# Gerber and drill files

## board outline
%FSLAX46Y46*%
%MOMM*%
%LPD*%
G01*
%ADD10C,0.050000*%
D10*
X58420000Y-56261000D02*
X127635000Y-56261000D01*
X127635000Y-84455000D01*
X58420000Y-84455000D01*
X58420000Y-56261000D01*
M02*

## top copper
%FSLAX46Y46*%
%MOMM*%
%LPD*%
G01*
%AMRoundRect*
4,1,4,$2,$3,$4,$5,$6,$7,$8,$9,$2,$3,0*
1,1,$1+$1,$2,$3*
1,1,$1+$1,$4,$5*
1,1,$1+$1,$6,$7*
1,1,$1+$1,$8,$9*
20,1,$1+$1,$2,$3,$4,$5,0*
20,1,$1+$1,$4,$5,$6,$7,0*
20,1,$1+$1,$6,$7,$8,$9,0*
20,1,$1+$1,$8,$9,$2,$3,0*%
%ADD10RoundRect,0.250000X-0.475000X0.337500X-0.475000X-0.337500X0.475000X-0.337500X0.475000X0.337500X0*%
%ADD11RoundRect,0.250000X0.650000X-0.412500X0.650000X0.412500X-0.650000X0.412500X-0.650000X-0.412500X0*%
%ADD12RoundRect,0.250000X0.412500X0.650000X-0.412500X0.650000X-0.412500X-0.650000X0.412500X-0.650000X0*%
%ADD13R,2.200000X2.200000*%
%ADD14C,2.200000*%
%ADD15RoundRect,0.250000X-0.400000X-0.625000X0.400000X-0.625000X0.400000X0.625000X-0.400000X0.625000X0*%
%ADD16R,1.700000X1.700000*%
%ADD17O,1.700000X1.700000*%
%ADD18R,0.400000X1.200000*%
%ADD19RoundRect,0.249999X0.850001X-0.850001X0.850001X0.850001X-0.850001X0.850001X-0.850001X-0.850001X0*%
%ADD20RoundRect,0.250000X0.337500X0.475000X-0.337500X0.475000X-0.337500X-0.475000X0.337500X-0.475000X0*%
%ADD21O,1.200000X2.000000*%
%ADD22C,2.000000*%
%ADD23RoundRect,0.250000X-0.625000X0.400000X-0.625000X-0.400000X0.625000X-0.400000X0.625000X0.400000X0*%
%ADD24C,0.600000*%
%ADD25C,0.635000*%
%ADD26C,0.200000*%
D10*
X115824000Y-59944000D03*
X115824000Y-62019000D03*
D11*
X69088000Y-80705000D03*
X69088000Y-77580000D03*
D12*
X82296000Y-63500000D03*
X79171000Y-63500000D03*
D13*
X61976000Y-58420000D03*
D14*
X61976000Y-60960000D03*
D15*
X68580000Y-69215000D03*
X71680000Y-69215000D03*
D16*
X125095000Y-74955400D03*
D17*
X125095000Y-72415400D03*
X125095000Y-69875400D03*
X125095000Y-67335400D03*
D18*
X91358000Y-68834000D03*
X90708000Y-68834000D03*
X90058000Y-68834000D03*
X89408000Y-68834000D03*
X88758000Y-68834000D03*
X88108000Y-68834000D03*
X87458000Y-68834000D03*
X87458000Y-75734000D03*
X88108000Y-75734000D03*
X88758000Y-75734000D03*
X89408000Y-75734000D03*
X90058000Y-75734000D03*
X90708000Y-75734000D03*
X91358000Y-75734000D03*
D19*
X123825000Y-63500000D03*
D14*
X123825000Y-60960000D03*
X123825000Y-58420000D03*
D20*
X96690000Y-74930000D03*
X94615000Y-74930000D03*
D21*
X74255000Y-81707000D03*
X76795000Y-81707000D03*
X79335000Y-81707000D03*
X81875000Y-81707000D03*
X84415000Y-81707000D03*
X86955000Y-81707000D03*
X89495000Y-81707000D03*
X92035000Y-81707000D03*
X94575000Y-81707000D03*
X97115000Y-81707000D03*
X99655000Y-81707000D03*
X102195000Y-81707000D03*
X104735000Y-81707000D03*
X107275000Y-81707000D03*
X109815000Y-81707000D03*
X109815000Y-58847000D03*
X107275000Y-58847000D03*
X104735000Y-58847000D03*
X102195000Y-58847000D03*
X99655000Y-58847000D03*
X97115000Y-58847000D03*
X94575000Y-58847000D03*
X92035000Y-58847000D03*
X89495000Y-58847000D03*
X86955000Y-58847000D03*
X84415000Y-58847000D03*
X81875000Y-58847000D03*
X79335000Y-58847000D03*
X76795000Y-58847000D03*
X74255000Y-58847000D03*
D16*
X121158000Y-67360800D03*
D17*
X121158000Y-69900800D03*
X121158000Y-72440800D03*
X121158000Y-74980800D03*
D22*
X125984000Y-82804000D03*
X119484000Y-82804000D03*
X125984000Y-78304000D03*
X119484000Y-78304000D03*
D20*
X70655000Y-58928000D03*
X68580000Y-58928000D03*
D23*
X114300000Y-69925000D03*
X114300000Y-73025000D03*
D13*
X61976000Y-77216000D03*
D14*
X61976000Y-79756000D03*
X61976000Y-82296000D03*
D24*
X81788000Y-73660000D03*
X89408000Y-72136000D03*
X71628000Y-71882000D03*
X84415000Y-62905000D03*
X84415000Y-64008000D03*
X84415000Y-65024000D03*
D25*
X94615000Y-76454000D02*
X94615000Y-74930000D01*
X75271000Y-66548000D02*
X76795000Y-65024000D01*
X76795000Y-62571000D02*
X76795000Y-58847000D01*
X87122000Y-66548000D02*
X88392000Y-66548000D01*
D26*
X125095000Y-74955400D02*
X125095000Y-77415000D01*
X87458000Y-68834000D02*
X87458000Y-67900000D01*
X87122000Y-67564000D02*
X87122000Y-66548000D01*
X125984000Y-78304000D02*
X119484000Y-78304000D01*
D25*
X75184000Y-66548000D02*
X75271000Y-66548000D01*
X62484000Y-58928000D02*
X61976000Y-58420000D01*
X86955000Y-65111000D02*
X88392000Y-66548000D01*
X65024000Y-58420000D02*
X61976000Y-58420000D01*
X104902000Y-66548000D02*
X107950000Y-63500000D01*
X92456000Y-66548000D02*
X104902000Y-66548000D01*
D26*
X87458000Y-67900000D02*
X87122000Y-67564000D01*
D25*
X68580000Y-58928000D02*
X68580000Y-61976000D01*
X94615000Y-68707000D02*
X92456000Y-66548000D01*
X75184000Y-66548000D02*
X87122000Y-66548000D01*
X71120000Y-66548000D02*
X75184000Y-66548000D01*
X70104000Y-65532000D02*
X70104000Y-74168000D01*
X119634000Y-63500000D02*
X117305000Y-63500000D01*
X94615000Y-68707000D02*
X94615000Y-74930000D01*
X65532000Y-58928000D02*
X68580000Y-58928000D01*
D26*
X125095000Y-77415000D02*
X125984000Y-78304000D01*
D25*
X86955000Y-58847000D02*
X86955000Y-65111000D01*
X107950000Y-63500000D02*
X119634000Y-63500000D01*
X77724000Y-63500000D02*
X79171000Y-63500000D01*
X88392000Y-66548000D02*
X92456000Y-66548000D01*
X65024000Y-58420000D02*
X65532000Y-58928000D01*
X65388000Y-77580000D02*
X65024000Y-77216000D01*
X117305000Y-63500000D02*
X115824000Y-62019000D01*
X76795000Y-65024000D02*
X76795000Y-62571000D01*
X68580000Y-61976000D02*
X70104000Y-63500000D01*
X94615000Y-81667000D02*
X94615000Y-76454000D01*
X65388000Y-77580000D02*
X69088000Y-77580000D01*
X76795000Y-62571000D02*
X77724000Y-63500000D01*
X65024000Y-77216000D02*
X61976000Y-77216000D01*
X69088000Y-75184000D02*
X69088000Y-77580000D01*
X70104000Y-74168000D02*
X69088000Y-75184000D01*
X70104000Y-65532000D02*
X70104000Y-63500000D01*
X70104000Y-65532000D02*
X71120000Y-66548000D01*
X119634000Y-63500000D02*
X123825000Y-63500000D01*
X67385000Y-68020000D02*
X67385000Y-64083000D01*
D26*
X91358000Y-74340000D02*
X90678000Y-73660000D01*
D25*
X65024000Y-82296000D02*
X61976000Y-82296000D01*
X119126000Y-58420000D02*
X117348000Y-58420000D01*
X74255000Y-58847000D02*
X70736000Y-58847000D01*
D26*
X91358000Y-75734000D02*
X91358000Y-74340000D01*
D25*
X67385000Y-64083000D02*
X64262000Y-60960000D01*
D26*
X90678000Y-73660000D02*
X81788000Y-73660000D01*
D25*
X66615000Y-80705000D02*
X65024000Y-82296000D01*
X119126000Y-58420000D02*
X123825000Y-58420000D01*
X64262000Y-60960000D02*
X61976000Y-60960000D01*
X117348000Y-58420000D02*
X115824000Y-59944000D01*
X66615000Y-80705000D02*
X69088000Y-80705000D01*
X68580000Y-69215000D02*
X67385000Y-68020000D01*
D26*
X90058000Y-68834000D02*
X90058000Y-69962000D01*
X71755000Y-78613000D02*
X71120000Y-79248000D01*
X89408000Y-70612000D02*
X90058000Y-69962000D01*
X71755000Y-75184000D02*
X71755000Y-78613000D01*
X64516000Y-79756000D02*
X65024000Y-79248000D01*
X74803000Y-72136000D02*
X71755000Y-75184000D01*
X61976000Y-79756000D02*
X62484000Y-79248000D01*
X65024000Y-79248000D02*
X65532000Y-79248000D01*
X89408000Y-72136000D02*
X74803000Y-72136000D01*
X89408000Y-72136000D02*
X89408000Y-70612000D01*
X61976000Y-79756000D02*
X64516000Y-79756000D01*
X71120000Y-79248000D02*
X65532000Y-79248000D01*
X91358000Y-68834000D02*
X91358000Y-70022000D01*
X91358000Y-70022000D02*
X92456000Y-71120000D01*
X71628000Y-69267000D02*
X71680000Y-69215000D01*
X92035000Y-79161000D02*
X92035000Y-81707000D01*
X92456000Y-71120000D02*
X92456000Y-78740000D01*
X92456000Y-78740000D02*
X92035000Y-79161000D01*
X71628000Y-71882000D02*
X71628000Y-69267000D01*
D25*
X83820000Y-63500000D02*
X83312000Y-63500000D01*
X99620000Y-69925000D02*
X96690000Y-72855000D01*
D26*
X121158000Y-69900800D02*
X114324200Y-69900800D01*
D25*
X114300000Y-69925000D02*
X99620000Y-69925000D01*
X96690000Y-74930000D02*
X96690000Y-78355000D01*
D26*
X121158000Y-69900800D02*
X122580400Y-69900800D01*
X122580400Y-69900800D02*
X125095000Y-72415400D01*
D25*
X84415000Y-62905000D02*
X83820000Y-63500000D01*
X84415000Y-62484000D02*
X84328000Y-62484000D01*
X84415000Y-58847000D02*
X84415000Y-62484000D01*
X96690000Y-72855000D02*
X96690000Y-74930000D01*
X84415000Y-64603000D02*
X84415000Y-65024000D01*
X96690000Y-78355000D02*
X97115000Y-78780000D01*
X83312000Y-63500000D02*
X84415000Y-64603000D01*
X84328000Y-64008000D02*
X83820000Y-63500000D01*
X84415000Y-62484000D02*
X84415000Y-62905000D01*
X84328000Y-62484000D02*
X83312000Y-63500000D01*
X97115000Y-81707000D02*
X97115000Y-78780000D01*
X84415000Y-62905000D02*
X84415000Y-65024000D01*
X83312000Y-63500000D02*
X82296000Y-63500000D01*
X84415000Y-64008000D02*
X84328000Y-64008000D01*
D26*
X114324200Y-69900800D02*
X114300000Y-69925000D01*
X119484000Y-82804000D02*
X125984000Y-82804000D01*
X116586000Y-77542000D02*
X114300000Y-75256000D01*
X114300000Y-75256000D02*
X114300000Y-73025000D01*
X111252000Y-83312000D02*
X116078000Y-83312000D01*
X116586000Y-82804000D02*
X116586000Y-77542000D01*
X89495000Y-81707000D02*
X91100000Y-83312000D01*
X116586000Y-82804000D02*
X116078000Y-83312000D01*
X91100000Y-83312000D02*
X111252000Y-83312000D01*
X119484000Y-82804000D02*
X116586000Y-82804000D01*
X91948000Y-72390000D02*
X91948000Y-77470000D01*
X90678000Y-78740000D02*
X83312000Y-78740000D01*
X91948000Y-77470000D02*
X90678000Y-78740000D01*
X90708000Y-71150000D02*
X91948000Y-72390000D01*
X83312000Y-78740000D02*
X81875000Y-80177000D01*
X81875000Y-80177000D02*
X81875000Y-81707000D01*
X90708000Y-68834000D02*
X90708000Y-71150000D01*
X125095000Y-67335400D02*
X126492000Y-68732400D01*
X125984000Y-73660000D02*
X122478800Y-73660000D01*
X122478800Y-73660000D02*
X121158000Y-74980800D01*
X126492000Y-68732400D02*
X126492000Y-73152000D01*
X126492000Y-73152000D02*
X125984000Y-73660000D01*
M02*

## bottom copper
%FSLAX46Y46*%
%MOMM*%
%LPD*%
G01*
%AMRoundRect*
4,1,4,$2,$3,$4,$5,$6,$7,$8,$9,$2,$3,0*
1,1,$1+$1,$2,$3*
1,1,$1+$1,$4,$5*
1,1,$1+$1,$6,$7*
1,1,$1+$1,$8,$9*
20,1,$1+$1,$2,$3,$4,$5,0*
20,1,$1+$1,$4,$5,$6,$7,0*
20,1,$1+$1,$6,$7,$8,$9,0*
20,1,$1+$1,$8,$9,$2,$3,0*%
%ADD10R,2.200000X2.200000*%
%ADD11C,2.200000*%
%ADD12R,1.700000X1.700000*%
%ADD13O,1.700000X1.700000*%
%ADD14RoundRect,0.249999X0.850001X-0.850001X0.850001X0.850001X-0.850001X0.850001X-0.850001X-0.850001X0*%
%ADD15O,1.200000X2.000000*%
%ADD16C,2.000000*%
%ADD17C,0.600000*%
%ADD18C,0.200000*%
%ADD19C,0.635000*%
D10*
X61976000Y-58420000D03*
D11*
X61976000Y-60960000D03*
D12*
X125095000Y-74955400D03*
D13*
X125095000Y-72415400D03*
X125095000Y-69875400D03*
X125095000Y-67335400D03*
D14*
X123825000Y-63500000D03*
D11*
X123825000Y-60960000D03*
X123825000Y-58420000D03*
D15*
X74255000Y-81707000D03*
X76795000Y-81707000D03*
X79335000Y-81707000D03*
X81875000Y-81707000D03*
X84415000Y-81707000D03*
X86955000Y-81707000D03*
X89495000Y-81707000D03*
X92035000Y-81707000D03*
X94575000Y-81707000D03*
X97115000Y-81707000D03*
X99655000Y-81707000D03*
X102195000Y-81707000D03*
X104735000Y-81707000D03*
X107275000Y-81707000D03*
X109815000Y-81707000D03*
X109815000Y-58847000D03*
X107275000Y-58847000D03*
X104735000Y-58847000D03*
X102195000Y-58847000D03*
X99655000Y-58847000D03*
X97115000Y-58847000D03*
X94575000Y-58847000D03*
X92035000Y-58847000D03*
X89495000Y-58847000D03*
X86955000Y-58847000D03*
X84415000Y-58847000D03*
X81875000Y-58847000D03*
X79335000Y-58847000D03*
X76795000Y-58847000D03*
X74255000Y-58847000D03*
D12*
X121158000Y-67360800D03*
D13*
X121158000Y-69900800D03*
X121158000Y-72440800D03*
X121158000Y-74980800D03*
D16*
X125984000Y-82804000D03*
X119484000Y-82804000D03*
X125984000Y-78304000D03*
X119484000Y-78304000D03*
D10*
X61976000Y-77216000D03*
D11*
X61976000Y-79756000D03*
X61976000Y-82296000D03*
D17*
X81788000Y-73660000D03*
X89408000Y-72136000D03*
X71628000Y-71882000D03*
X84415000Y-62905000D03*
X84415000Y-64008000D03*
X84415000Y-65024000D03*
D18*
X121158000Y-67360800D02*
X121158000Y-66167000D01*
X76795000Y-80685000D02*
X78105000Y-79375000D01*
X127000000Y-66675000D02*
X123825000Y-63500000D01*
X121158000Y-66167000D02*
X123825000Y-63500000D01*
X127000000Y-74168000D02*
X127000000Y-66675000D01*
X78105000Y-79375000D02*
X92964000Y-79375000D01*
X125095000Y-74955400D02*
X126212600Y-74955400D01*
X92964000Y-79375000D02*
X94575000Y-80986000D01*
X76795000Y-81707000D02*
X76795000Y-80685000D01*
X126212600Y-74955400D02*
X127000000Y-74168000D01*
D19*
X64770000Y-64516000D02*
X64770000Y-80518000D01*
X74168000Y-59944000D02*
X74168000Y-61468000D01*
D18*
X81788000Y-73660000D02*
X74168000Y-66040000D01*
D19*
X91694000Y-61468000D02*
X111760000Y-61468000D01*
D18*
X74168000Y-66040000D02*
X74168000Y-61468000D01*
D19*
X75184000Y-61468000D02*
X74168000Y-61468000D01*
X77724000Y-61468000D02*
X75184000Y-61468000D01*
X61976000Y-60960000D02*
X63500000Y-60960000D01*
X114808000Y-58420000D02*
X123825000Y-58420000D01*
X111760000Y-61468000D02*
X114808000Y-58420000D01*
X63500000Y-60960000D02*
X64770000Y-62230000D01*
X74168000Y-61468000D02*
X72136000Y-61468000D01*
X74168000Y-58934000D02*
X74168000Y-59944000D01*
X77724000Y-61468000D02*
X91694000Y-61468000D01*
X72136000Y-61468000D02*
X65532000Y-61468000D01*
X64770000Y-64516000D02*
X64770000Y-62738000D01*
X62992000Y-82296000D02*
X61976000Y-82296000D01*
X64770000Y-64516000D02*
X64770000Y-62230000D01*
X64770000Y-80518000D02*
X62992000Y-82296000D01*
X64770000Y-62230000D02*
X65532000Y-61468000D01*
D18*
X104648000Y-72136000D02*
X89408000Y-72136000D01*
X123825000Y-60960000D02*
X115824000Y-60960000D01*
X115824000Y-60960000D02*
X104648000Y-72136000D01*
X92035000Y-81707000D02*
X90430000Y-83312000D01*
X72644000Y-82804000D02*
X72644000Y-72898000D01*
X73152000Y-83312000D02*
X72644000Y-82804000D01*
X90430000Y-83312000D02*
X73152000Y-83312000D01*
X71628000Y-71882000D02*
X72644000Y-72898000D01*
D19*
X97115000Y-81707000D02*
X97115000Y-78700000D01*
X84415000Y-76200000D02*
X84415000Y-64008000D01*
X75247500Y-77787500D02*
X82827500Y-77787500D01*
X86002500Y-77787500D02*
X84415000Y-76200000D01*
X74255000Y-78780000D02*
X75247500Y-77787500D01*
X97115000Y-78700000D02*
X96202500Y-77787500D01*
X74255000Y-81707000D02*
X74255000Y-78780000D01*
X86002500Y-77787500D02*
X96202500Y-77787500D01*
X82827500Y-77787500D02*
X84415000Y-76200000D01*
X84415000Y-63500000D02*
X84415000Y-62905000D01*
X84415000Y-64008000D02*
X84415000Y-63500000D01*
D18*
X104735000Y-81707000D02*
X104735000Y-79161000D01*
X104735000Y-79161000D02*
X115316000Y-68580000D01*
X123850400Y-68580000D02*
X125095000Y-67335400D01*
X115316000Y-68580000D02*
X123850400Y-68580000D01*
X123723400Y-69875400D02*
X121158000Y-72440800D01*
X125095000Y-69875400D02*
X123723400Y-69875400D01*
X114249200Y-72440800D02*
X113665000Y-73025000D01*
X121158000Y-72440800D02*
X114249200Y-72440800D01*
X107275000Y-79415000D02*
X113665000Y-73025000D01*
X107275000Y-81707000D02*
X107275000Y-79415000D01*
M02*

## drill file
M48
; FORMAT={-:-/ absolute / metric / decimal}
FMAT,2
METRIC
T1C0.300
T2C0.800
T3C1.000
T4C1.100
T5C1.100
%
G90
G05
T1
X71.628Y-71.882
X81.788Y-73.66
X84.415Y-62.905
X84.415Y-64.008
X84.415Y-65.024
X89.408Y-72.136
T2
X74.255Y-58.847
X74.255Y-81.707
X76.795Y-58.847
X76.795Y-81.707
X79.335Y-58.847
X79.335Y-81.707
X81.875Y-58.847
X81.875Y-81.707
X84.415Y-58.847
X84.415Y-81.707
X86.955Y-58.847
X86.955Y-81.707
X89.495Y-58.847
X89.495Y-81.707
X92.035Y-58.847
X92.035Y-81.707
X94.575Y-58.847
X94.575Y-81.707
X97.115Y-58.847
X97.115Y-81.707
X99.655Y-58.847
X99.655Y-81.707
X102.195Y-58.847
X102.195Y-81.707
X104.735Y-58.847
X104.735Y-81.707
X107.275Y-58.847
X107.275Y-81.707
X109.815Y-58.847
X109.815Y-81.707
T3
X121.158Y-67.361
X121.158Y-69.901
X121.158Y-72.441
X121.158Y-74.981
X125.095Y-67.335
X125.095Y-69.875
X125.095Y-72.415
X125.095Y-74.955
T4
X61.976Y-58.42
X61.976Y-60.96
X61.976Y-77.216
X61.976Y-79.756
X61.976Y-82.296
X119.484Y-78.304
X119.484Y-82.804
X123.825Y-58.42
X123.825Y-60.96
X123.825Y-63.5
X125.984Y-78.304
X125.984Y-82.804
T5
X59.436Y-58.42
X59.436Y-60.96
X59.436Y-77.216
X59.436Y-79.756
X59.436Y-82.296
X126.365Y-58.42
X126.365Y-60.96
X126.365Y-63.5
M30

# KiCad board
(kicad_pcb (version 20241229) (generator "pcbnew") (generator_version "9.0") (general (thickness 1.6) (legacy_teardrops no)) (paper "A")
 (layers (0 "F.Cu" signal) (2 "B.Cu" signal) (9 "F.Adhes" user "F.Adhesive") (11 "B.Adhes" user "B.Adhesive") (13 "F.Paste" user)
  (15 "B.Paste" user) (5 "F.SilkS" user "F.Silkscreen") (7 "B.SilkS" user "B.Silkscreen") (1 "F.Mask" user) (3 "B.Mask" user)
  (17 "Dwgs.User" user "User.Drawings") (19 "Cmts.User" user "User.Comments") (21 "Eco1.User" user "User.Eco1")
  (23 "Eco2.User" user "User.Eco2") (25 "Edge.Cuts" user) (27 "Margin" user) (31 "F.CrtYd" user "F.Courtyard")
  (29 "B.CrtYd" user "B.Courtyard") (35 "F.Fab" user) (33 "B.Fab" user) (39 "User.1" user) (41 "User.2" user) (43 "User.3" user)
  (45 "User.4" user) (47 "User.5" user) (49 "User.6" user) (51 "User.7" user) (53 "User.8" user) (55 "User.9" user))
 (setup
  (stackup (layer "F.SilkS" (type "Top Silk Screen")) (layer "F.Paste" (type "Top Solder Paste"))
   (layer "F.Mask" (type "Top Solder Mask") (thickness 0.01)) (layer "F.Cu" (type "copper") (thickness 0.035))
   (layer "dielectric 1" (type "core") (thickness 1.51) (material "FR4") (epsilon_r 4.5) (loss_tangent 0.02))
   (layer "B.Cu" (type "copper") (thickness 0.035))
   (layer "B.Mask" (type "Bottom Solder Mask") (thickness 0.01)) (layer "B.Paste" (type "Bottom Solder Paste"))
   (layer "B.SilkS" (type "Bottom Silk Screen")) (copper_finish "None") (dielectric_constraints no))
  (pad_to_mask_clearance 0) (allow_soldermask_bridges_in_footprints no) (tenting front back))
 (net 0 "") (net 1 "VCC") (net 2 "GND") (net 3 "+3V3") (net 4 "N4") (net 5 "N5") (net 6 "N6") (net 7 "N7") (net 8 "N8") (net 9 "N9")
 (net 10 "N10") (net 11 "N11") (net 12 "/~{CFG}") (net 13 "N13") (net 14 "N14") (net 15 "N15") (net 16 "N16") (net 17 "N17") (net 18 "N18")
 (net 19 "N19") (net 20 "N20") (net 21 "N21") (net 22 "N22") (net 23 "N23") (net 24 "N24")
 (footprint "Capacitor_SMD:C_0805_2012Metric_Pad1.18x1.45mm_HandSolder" (layer "F.Cu") (at 115.824 60.9815 -90)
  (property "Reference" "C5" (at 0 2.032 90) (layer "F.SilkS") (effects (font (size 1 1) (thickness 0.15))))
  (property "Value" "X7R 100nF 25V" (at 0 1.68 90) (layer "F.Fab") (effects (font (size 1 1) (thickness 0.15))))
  (pad "1" smd roundrect (at -1.0375 0 270) (size 1.175 1.45) (layers "F.Cu" "F.Mask" "F.Paste") (roundrect_rratio 0.212766) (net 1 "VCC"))
  (pad "2" smd roundrect (at 1.0375 0 270) (size 1.175 1.45) (layers "F.Cu" "F.Mask" "F.Paste") (roundrect_rratio 0.212766) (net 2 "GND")))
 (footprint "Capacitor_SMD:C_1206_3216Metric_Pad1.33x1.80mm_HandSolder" (layer "F.Cu") (at 69.088 79.1425 90)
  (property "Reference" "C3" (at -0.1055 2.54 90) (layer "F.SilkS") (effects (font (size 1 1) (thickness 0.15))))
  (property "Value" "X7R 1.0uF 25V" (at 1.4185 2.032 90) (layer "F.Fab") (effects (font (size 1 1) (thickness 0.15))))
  (pad "1" smd roundrect (at -1.5625 0 90) (size 1.325 1.8) (layers "F.Cu" "F.Mask" "F.Paste") (roundrect_rratio 0.188679) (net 1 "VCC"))
  (pad "2" smd roundrect (at 1.5625 0 90) (size 1.325 1.8) (layers "F.Cu" "F.Mask" "F.Paste") (roundrect_rratio 0.188679) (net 2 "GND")))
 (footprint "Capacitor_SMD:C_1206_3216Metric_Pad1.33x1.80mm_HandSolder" (layer "F.Cu") (at 80.7335 63.5 180)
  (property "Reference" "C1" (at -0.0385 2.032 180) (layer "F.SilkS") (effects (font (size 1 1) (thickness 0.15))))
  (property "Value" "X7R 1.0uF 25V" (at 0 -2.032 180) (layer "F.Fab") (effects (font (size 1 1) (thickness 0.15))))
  (pad "1" smd roundrect (at -1.5625 0 180) (size 1.325 1.8) (layers "F.Cu" "F.Mask" "F.Paste") (roundrect_rratio 0.188679) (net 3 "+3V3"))
  (pad "2" smd roundrect (at 1.5625 0 180) (size 1.325 1.8) (layers "F.Cu" "F.Mask" "F.Paste") (roundrect_rratio 0.188679) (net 2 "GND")))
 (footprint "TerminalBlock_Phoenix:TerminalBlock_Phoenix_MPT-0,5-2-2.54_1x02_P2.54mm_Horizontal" (layer "F.Cu") (at 61.976 58.42 -90)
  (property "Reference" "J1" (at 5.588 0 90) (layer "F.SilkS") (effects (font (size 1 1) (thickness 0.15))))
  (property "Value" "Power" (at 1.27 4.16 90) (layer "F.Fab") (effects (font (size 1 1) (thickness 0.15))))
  (pad "" np_thru_hole circle (at 0 2.54 270) (size 1.1 1.1) (drill 1.1) (layers "*.Cu" "*.Mask"))
  (pad "" np_thru_hole circle (at 2.54 2.54 270) (size 1.1 1.1) (drill 1.1) (layers "*.Cu" "*.Mask"))
  (pad "1" thru_hole rect (at 0 0 270) (size 2.2 2.2) (drill 1.1) (layers "*.Cu" "*.Mask") (remove_unused_layers no) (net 2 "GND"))
  (pad "2" thru_hole circle (at 2.54 0 270) (size 2.2 2.2) (drill 1.1) (layers "*.Cu" "*.Mask") (remove_unused_layers no) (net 1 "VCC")))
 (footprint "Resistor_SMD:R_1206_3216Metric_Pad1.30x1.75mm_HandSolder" (layer "F.Cu") (at 70.13 69.215)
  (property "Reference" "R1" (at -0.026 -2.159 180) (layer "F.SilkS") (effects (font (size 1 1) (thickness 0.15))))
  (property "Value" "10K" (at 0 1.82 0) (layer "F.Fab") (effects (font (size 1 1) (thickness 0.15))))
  (pad "1" smd roundrect (at -1.55 0) (size 1.3 1.75) (layers "F.Cu" "F.Mask" "F.Paste") (roundrect_rratio 0.192308) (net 1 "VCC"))
  (pad "2" smd roundrect (at 1.55 0) (size 1.3 1.75) (layers "F.Cu" "F.Mask" "F.Paste") (roundrect_rratio 0.192308) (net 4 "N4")))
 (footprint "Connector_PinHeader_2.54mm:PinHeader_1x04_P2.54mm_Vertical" (layer "F.Cu") (at 125.095 74.9554 180)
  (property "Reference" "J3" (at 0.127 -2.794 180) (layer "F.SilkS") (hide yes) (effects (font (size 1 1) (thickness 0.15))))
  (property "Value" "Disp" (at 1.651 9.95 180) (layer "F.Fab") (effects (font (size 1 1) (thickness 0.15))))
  (pad "1" thru_hole rect (at 0 0 180) (size 1.7 1.7) (drill 1) (layers "*.Cu" "*.Mask") (remove_unused_layers no) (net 2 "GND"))
  (pad "2" thru_hole oval (at 0 2.54 180) (size 1.7 1.7) (drill 1) (layers "*.Cu" "*.Mask") (remove_unused_layers no) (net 3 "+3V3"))
  (pad "3" thru_hole oval (at 0 5.08 180) (size 1.7 1.7) (drill 1) (layers "*.Cu" "*.Mask") (remove_unused_layers no) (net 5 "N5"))
  (pad "4" thru_hole oval (at 0 7.62 180) (size 1.7 1.7) (drill 1) (layers "*.Cu" "*.Mask") (remove_unused_layers no) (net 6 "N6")))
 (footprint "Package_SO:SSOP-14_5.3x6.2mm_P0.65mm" (layer "F.Cu") (at 89.408 72.284 -90)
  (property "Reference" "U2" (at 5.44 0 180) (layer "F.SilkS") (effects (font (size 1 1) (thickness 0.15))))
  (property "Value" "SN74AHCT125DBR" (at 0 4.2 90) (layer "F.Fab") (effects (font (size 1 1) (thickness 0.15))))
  (pad "1" smd rect (at -3.45 -1.95 270) (size 1.2 0.4) (layers "F.Cu" "F.Mask" "F.Paste") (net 4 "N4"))
  (pad "2" smd rect (at -3.45 -1.3 270) (size 1.2 0.4) (layers "F.Cu" "F.Mask" "F.Paste") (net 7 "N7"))
  (pad "3" smd rect (at -3.45 -0.65 270) (size 1.2 0.4) (layers "F.Cu" "F.Mask" "F.Paste") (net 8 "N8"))
  (pad "4" smd rect (at -3.45 0 270) (size 1.2 0.4) (layers "F.Cu" "F.Mask" "F.Paste"))
  (pad "5" smd rect (at -3.45 0.65 270) (size 1.2 0.4) (layers "F.Cu" "F.Mask" "F.Paste"))
  (pad "6" smd rect (at -3.45 1.3 270) (size 1.2 0.4) (layers "F.Cu" "F.Mask" "F.Paste"))
  (pad "7" smd rect (at -3.45 1.95 270) (size 1.2 0.4) (layers "F.Cu" "F.Mask" "F.Paste") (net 2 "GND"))
  (pad "8" smd rect (at 3.45 1.95 270) (size 1.2 0.4) (layers "F.Cu" "F.Mask" "F.Paste"))
  (pad "9" smd rect (at 3.45 1.3 270) (size 1.2 0.4) (layers "F.Cu" "F.Mask" "F.Paste"))
  (pad "10" smd rect (at 3.45 0.65 270) (size 1.2 0.4) (layers "F.Cu" "F.Mask" "F.Paste"))
  (pad "11" smd rect (at 3.45 0 270) (size 1.2 0.4) (layers "F.Cu" "F.Mask" "F.Paste"))
  (pad "12" smd rect (at 3.45 -0.65 270) (size 1.2 0.4) (layers "F.Cu" "F.Mask" "F.Paste"))
  (pad "13" smd rect (at 3.45 -1.3 270) (size 1.2 0.4) (layers "F.Cu" "F.Mask" "F.Paste"))
  (pad "14" smd rect (at 3.45 -1.95 270) (size 1.2 0.4) (layers "F.Cu" "F.Mask" "F.Paste") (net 1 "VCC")))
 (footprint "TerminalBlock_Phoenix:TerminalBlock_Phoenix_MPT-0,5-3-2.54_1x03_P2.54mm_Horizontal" (layer "F.Cu") (at 123.825 63.5 90)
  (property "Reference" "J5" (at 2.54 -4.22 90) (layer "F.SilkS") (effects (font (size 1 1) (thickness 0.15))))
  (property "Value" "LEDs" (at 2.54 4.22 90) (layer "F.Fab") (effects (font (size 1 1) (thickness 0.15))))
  (pad "" np_thru_hole circle (at 0 2.54 90) (size 1.1 1.1) (drill 1.1) (layers "*.Cu" "*.Mask"))
  (pad "" np_thru_hole circle (at 2.54 2.54 90) (size 1.1 1.1) (drill 1.1) (layers "*.Cu" "*.Mask"))
  (pad "" np_thru_hole circle (at 5.08 2.54 90) (size 1.1 1.1) (drill 1.1) (layers "*.Cu" "*.Mask"))
  (pad "1" thru_hole roundrect (at 0 0 90) (size 2.2 2.2) (drill 1.1) (layers "*.Cu" "*.Mask") (remove_unused_layers no)
   (roundrect_rratio 0.113636) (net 2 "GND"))
  (pad "2" thru_hole circle (at 2.54 0 90) (size 2.2 2.2) (drill 1.1) (layers "*.Cu" "*.Mask") (remove_unused_layers no) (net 8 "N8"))
  (pad "3" thru_hole circle (at 5.08 0 90) (size 2.2 2.2) (drill 1.1) (layers "*.Cu" "*.Mask") (remove_unused_layers no) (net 1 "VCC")))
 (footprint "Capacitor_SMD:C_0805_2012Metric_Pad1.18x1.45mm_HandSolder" (layer "F.Cu") (at 95.6525 74.93 180)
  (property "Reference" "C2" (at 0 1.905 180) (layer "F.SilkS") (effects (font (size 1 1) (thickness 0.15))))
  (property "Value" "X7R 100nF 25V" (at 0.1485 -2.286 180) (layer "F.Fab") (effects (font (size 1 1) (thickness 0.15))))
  (pad "1" smd roundrect (at -1.0375 0 180) (size 1.175 1.45) (layers "F.Cu" "F.Mask" "F.Paste") (roundrect_rratio 0.212766) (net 3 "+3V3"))
  (pad "2" smd roundrect (at 1.0375 0 180) (size 1.175 1.45) (layers "F.Cu" "F.Mask" "F.Paste") (roundrect_rratio 0.212766) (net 2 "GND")))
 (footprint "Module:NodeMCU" (layer "F.Cu") (at 92.035 70.277)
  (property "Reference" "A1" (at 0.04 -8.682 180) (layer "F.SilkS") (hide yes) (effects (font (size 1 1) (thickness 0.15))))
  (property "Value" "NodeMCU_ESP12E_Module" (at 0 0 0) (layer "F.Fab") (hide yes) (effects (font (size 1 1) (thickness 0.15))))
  (pad "1" thru_hole oval (at -17.78 11.43) (size 1.2 2) (drill 0.8) (layers "*.Cu" "*.Mask") (remove_unused_layers no) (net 3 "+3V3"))
  (pad "2" thru_hole oval (at -15.24 11.43) (size 1.2 2) (drill 0.8) (layers "*.Cu" "*.Mask") (remove_unused_layers no) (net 2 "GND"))
  (pad "3" thru_hole oval (at -12.7 11.43) (size 1.2 2) (drill 0.8) (layers "*.Cu" "*.Mask") (remove_unused_layers no) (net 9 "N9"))
  (pad "4" thru_hole oval (at -10.16 11.43) (size 1.2 2) (drill 0.8) (layers "*.Cu" "*.Mask") (remove_unused_layers no) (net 7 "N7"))
  (pad "5" thru_hole oval (at -7.62 11.43) (size 1.2 2) (drill 0.8) (layers "*.Cu" "*.Mask") (remove_unused_layers no) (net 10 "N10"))
  (pad "6" thru_hole oval (at -5.08 11.43) (size 1.2 2) (drill 0.8) (layers "*.Cu" "*.Mask") (remove_unused_layers no) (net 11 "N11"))
  (pad "7" thru_hole oval (at -2.54 11.43) (size 1.2 2) (drill 0.8) (layers "*.Cu" "*.Mask") (remove_unused_layers no) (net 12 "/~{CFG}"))
  (pad "8" thru_hole oval (at 0 11.43) (size 1.2 2) (drill 0.8) (layers "*.Cu" "*.Mask") (remove_unused_layers no) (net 4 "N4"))
  (pad "9" thru_hole oval (at 2.54 11.43) (size 1.2 2) (drill 0.8) (layers "*.Cu" "*.Mask") (remove_unused_layers no) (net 2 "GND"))
  (pad "10" thru_hole oval (at 5.08 11.43) (size 1.2 2) (drill 0.8) (layers "*.Cu" "*.Mask") (remove_unused_layers no) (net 3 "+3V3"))
  (pad "11" thru_hole oval (at 7.62 11.43) (size 1.2 2) (drill 0.8) (layers "*.Cu" "*.Mask") (remove_unused_layers no) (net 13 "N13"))
  (pad "12" thru_hole oval (at 10.16 11.43) (size 1.2 2) (drill 0.8) (layers "*.Cu" "*.Mask") (remove_unused_layers no) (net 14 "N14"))
  (pad "13" thru_hole oval (at 12.7 11.43) (size 1.2 2) (drill 0.8) (layers "*.Cu" "*.Mask") (remove_unused_layers no) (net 6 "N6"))
  (pad "14" thru_hole oval (at 15.24 11.43) (size 1.2 2) (drill 0.8) (layers "*.Cu" "*.Mask") (remove_unused_layers no) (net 5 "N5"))
  (pad "15" thru_hole oval (at 17.78 11.43) (size 1.2 2) (drill 0.8) (layers "*.Cu" "*.Mask") (remove_unused_layers no) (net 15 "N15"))
  (pad "16" thru_hole oval (at 17.78 -11.43) (size 1.2 2) (drill 0.8) (layers "*.Cu" "*.Mask") (remove_unused_layers no) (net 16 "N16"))
  (pad "17" thru_hole oval (at 15.24 -11.43) (size 1.2 2) (drill 0.8) (layers "*.Cu" "*.Mask") (remove_unused_layers no))
  (pad "18" thru_hole oval (at 12.7 -11.43) (size 1.2 2) (drill 0.8) (layers "*.Cu" "*.Mask") (remove_unused_layers no))
  (pad "19" thru_hole oval (at 10.16 -11.43) (size 1.2 2) (drill 0.8) (layers "*.Cu" "*.Mask") (remove_unused_layers no) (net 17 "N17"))
  (pad "20" thru_hole oval (at 7.62 -11.43) (size 1.2 2) (drill 0.8) (layers "*.Cu" "*.Mask") (remove_unused_layers no) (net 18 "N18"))
  (pad "21" thru_hole oval (at 5.08 -11.43) (size 1.2 2) (drill 0.8) (layers "*.Cu" "*.Mask") (remove_unused_layers no) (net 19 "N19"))
  (pad "22" thru_hole oval (at 2.54 -11.43) (size 1.2 2) (drill 0.8) (layers "*.Cu" "*.Mask") (remove_unused_layers no) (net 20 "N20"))
  (pad "23" thru_hole oval (at 0 -11.43) (size 1.2 2) (drill 0.8) (layers "*.Cu" "*.Mask") (remove_unused_layers no) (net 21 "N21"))
  (pad "24" thru_hole oval (at -2.54 -11.43) (size 1.2 2) (drill 0.8) (layers "*.Cu" "*.Mask") (remove_unused_layers no) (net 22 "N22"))
  (pad "25" thru_hole oval (at -5.08 -11.43) (size 1.2 2) (drill 0.8) (layers "*.Cu" "*.Mask") (remove_unused_layers no) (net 2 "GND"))
  (pad "26" thru_hole oval (at -7.62 -11.43) (size 1.2 2) (drill 0.8) (layers "*.Cu" "*.Mask") (remove_unused_layers no) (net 3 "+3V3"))
  (pad "27" thru_hole oval (at -10.16 -11.43) (size 1.2 2) (drill 0.8) (layers "*.Cu" "*.Mask") (remove_unused_layers no) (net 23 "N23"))
  (pad "28" thru_hole oval (at -12.7 -11.43) (size 1.2 2) (drill 0.8) (layers "*.Cu" "*.Mask") (remove_unused_layers no) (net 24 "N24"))
  (pad "29" thru_hole oval (at -15.24 -11.43) (size 1.2 2) (drill 0.8) (layers "*.Cu" "*.Mask") (remove_unused_layers no) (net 2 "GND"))
  (pad "30" thru_hole oval (at -17.78 -11.43) (size 1.2 2) (drill 0.8) (layers "*.Cu" "*.Mask") (remove_unused_layers no) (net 1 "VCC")))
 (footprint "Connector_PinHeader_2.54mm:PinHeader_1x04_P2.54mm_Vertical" (layer "F.Cu") (at 121.158 67.3608)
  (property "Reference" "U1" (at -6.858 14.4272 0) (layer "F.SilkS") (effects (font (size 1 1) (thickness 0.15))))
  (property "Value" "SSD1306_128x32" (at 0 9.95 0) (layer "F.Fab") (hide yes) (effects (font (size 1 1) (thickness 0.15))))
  (pad "1" thru_hole rect (at 0 0) (size 1.7 1.7) (drill 1) (layers "*.Cu" "*.Mask") (remove_unused_layers no) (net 2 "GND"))
  (pad "2" thru_hole oval (at 0 2.54) (size 1.7 1.7) (drill 1) (layers "*.Cu" "*.Mask") (remove_unused_layers no) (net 3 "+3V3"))
  (pad "3" thru_hole oval (at 0 5.08) (size 1.7 1.7) (drill 1) (layers "*.Cu" "*.Mask") (remove_unused_layers no) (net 5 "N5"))
  (pad "4" thru_hole oval (at 0 7.62) (size 1.7 1.7) (drill 1) (layers "*.Cu" "*.Mask") (remove_unused_layers no) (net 6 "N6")))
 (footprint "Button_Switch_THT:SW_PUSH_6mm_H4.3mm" (layer "F.Cu") (at 125.984 82.804 180)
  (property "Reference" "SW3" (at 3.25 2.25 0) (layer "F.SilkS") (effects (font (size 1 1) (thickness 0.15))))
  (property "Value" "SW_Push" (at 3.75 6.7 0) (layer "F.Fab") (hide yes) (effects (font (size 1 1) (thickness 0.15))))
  (pad "1" thru_hole circle (at 0 0 270) (size 2 2) (drill 1.1) (layers "*.Cu" "*.Mask") (remove_unused_layers no) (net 12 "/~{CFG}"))
  (pad "1" thru_hole circle (at 6.5 0 270) (size 2 2) (drill 1.1) (layers "*.Cu" "*.Mask") (remove_unused_layers no) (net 12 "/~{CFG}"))
  (pad "2" thru_hole circle (at 0 4.5 270) (size 2 2) (drill 1.1) (layers "*.Cu" "*.Mask") (remove_unused_layers no) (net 2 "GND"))
  (pad "2" thru_hole circle (at 6.5 4.5 270) (size 2 2) (drill 1.1) (layers "*.Cu" "*.Mask") (remove_unused_layers no) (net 2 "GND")))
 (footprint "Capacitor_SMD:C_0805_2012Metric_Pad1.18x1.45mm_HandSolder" (layer "F.Cu") (at 69.6175 58.928 180)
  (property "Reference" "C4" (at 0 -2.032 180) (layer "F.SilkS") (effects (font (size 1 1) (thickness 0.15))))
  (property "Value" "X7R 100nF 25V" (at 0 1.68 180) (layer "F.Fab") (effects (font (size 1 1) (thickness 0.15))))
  (pad "1" smd roundrect (at -1.0375 0 180) (size 1.175 1.45) (layers "F.Cu" "F.Mask" "F.Paste") (roundrect_rratio 0.212766) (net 1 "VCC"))
  (pad "2" smd roundrect (at 1.0375 0 180) (size 1.175 1.45) (layers "F.Cu" "F.Mask" "F.Paste") (roundrect_rratio 0.212766) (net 2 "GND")))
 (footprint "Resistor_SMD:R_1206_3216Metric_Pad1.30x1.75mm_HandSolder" (layer "F.Cu") (at 114.3 71.475 -90)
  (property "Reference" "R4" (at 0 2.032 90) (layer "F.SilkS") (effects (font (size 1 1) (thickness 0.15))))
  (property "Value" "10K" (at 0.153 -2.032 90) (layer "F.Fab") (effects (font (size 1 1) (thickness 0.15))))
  (pad "1" smd roundrect (at -1.55 0 270) (size 1.3 1.75) (layers "F.Cu" "F.Mask" "F.Paste") (roundrect_rratio 0.192308) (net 3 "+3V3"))
  (pad "2" smd roundrect (at 1.55 0 270) (size 1.3 1.75) (layers "F.Cu" "F.Mask" "F.Paste") (roundrect_rratio 0.192308) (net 12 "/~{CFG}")))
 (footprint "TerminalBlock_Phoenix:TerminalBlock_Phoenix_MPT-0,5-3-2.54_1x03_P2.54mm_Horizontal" (layer "F.Cu") (at 61.976 77.216 -90)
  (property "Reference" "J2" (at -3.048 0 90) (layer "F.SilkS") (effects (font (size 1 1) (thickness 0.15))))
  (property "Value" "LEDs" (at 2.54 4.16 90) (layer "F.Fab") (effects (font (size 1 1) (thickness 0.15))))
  (pad "" np_thru_hole circle (at 0 2.54 270) (size 1.1 1.1) (drill 1.1) (layers "*.Cu" "*.Mask"))
  (pad "" np_thru_hole circle (at 2.54 2.54 270) (size 1.1 1.1) (drill 1.1) (layers "*.Cu" "*.Mask"))
  (pad "" np_thru_hole circle (at 5.08 2.54 270) (size 1.1 1.1) (drill 1.1) (layers "*.Cu" "*.Mask"))
  (pad "1" thru_hole rect (at 0 0 270) (size 2.2 2.2) (drill 1.1) (layers "*.Cu" "*.Mask") (remove_unused_layers no) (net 2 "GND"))
  (pad "2" thru_hole circle (at 2.54 0 270) (size 2.2 2.2) (drill 1.1) (layers "*.Cu" "*.Mask") (remove_unused_layers no) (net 8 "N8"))
  (pad "3" thru_hole circle (at 5.08 0 270) (size 2.2 2.2) (drill 1.1) (layers "*.Cu" "*.Mask") (remove_unused_layers no) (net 1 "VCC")))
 (gr_rect (start 58.42 56.261) (end 127.635 84.455) (stroke (width 0.05) (type default)) (fill no) (layer "Edge.Cuts"))
 (segment (start 94.615 76.454) (end 94.615 74.93) (width 0.635) (layer "F.Cu") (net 2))
 (segment (start 75.271 66.548) (end 76.795 65.024) (width 0.635) (layer "F.Cu") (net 2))
 (segment (start 76.795 62.571) (end 76.795 58.847) (width 0.635) (layer "F.Cu") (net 2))
 (segment (start 87.122 66.548) (end 88.392 66.548) (width 0.635) (layer "F.Cu") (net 2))
 (segment (start 125.095 74.9554) (end 125.095 77.415) (width 0.2) (layer "F.Cu") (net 2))
 (segment (start 87.458 68.834) (end 87.458 67.9) (width 0.2) (layer "F.Cu") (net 2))
 (segment (start 87.122 67.564) (end 87.122 66.548) (width 0.2) (layer "F.Cu") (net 2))
 (segment (start 125.984 78.304) (end 119.484 78.304) (width 0.2) (layer "F.Cu") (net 2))
 (segment (start 75.184 66.548) (end 75.271 66.548) (width 0.635) (layer "F.Cu") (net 2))
 (segment (start 62.484 58.928) (end 61.976 58.42) (width 0.635) (layer "F.Cu") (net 2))
 (segment (start 86.955 65.111) (end 88.392 66.548) (width 0.635) (layer "F.Cu") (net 2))
 (segment (start 65.024 58.42) (end 61.976 58.42) (width 0.635) (layer "F.Cu") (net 2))
 (segment (start 104.902 66.548) (end 107.95 63.5) (width 0.635) (layer "F.Cu") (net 2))
 (segment (start 92.456 66.548) (end 104.902 66.548) (width 0.635) (layer "F.Cu") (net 2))
 (segment (start 87.458 67.9) (end 87.122 67.564) (width 0.2) (layer "F.Cu") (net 2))
 (segment (start 68.58 58.928) (end 68.58 61.976) (width 0.635) (layer "F.Cu") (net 2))
 (segment (start 94.615 68.707) (end 92.456 66.548) (width 0.635) (layer "F.Cu") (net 2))
 (segment (start 75.184 66.548) (end 87.122 66.548) (width 0.635) (layer "F.Cu") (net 2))
 (segment (start 71.12 66.548) (end 75.184 66.548) (width 0.635) (layer "F.Cu") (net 2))
 (segment (start 70.104 65.532) (end 70.104 74.168) (width 0.635) (layer "F.Cu") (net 2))
 (segment (start 119.634 63.5) (end 117.305 63.5) (width 0.635) (layer "F.Cu") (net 2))
 (segment (start 94.615 68.707) (end 94.615 74.93) (width 0.635) (layer "F.Cu") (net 2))
 (segment (start 65.532 58.928) (end 68.58 58.928) (width 0.635) (layer "F.Cu") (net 2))
 (segment (start 125.095 77.415) (end 125.984 78.304) (width 0.2) (layer "F.Cu") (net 2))
 (segment (start 86.955 58.847) (end 86.955 65.111) (width 0.635) (layer "F.Cu") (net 2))
 (segment (start 107.95 63.5) (end 119.634 63.5) (width 0.635) (layer "F.Cu") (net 2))
 (segment (start 77.724 63.5) (end 79.171 63.5) (width 0.635) (layer "F.Cu") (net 2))
 (segment (start 88.392 66.548) (end 92.456 66.548) (width 0.635) (layer "F.Cu") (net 2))
 (segment (start 65.024 58.42) (end 65.532 58.928) (width 0.635) (layer "F.Cu") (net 2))
 (segment (start 65.388 77.58) (end 65.024 77.216) (width 0.635) (layer "F.Cu") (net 2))
 (segment (start 117.305 63.5) (end 115.824 62.019) (width 0.635) (layer "F.Cu") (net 2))
 (segment (start 76.795 65.024) (end 76.795 62.571) (width 0.635) (layer "F.Cu") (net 2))
 (segment (start 68.58 61.976) (end 70.104 63.5) (width 0.635) (layer "F.Cu") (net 2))
 (segment (start 94.615 81.667) (end 94.615 76.454) (width 0.635) (layer "F.Cu") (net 2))
 (segment (start 65.388 77.58) (end 69.088 77.58) (width 0.635) (layer "F.Cu") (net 2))
 (segment (start 76.795 62.571) (end 77.724 63.5) (width 0.635) (layer "F.Cu") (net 2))
 (segment (start 65.024 77.216) (end 61.976 77.216) (width 0.635) (layer "F.Cu") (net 2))
 (segment (start 69.088 75.184) (end 69.088 77.58) (width 0.635) (layer "F.Cu") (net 2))
 (segment (start 70.104 74.168) (end 69.088 75.184) (width 0.635) (layer "F.Cu") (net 2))
 (segment (start 70.104 65.532) (end 70.104 63.5) (width 0.635) (layer "F.Cu") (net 2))
 (segment (start 70.104 65.532) (end 71.12 66.548) (width 0.635) (layer "F.Cu") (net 2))
 (segment (start 119.634 63.5) (end 123.825 63.5) (width 0.635) (layer "F.Cu") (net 2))
 (segment (start 121.158 67.3608) (end 121.158 66.167) (width 0.2) (layer "B.Cu") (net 2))
 (segment (start 76.795 80.685) (end 78.105 79.375) (width 0.2) (layer "B.Cu") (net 2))
 (segment (start 127 66.675) (end 123.825 63.5) (width 0.2) (layer "B.Cu") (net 2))
 (segment (start 121.158 66.167) (end 123.825 63.5) (width 0.2) (layer "B.Cu") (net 2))
 (segment (start 127 74.168) (end 127 66.675) (width 0.2) (layer "B.Cu") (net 2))
 (segment (start 78.105 79.375) (end 92.964 79.375) (width 0.2) (layer "B.Cu") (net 2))
 (segment (start 125.095 74.9554) (end 126.2126 74.9554) (width 0.2) (layer "B.Cu") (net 2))
 (segment (start 92.964 79.375) (end 94.575 80.986) (width 0.2) (layer "B.Cu") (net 2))
 (segment (start 76.795 81.707) (end 76.795 80.685) (width 0.2) (layer "B.Cu") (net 2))
 (segment (start 126.2126 74.9554) (end 127 74.168) (width 0.2) (layer "B.Cu") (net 2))
 (segment (start 67.385 68.02) (end 67.385 64.083) (width 0.635) (layer "F.Cu") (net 1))
 (segment (start 91.358 74.34) (end 90.678 73.66) (width 0.2) (layer "F.Cu") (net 1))
 (segment (start 65.024 82.296) (end 61.976 82.296) (width 0.635) (layer "F.Cu") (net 1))
 (segment (start 119.126 58.42) (end 117.348 58.42) (width 0.635) (layer "F.Cu") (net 1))
 (segment (start 74.255 58.847) (end 70.736 58.847) (width 0.635) (layer "F.Cu") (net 1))
 (segment (start 91.358 75.734) (end 91.358 74.34) (width 0.2) (layer "F.Cu") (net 1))
 (segment (start 67.385 64.083) (end 64.262 60.96) (width 0.635) (layer "F.Cu") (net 1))
 (segment (start 90.678 73.66) (end 81.788 73.66) (width 0.2) (layer "F.Cu") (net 1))
 (segment (start 66.615 80.705) (end 65.024 82.296) (width 0.635) (layer "F.Cu") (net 1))
 (segment (start 119.126 58.42) (end 123.825 58.42) (width 0.635) (layer "F.Cu") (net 1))
 (segment (start 64.262 60.96) (end 61.976 60.96) (width 0.635) (layer "F.Cu") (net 1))
 (segment (start 117.348 58.42) (end 115.824 59.944) (width 0.635) (layer "F.Cu") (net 1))
 (segment (start 66.615 80.705) (end 69.088 80.705) (width 0.635) (layer "F.Cu") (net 1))
 (segment (start 68.58 69.215) (end 67.385 68.02) (width 0.635) (layer "F.Cu") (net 1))
 (via (at 81.788 73.66) (size 0.6) (drill 0.3) (layers "F.Cu" "B.Cu") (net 1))
 (segment (start 64.77 64.516) (end 64.77 80.518) (width 0.635) (layer "B.Cu") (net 1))
 (segment (start 74.168 59.944) (end 74.168 61.468) (width 0.635) (layer "B.Cu") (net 1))
 (segment (start 81.788 73.66) (end 74.168 66.04) (width 0.2) (layer "B.Cu") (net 1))
 (segment (start 91.694 61.468) (end 111.76 61.468) (width 0.635) (layer "B.Cu") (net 1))
 (segment (start 74.168 66.04) (end 74.168 61.468) (width 0.2) (layer "B.Cu") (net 1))
 (segment (start 75.184 61.468) (end 74.168 61.468) (width 0.635) (layer "B.Cu") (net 1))
 (segment (start 77.724 61.468) (end 75.184 61.468) (width 0.635) (layer "B.Cu") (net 1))
 (segment (start 61.976 60.96) (end 63.5 60.96) (width 0.635) (layer "B.Cu") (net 1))
 (segment (start 114.808 58.42) (end 123.825 58.42) (width 0.635) (layer "B.Cu") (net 1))
 (segment (start 111.76 61.468) (end 114.808 58.42) (width 0.635) (layer "B.Cu") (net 1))
 (segment (start 63.5 60.96) (end 64.77 62.23) (width 0.635) (layer "B.Cu") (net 1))
 (segment (start 74.168 61.468) (end 72.136 61.468) (width 0.635) (layer "B.Cu") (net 1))
 (segment (start 74.168 58.934) (end 74.168 59.944) (width 0.635) (layer "B.Cu") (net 1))
 (segment (start 77.724 61.468) (end 91.694 61.468) (width 0.635) (layer "B.Cu") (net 1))
 (segment (start 72.136 61.468) (end 65.532 61.468) (width 0.635) (layer "B.Cu") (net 1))
 (segment (start 64.77 64.516) (end 64.77 62.738) (width 0.635) (layer "B.Cu") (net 1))
 (segment (start 62.992 82.296) (end 61.976 82.296) (width 0.635) (layer "B.Cu") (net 1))
 (segment (start 64.77 64.516) (end 64.77 62.23) (width 0.635) (layer "B.Cu") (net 1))
 (segment (start 64.77 80.518) (end 62.992 82.296) (width 0.635) (layer "B.Cu") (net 1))
 (segment (start 64.77 62.23) (end 65.532 61.468) (width 0.635) (layer "B.Cu") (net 1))
 (segment (start 90.058 68.834) (end 90.058 69.962) (width 0.2) (layer "F.Cu") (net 8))
 (segment (start 71.755 78.613) (end 71.12 79.248) (width 0.2) (layer "F.Cu") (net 8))
 (segment (start 89.408 70.612) (end 90.058 69.962) (width 0.2) (layer "F.Cu") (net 8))
 (segment (start 71.755 75.184) (end 71.755 78.613) (width 0.2) (layer "F.Cu") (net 8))
 (segment (start 64.516 79.756) (end 65.024 79.248) (width 0.2) (layer "F.Cu") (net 8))
 (segment (start 74.803 72.136) (end 71.755 75.184) (width 0.2) (layer "F.Cu") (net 8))
 (segment (start 61.976 79.756) (end 62.484 79.248) (width 0.2) (layer "F.Cu") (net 8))
 (segment (start 65.024 79.248) (end 65.532 79.248) (width 0.2) (layer "F.Cu") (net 8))
 (segment (start 89.408 72.136) (end 74.803 72.136) (width 0.2) (layer "F.Cu") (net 8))
 (segment (start 89.408 72.136) (end 89.408 70.612) (width 0.2) (layer "F.Cu") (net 8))
 (segment (start 61.976 79.756) (end 64.516 79.756) (width 0.2) (layer "F.Cu") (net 8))
 (segment (start 71.12 79.248) (end 65.532 79.248) (width 0.2) (layer "F.Cu") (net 8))
 (via (at 89.408 72.136) (size 0.6) (drill 0.3) (layers "F.Cu" "B.Cu") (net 8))
 (segment (start 104.648 72.136) (end 89.408 72.136) (width 0.2) (layer "B.Cu") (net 8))
 (segment (start 123.825 60.96) (end 115.824 60.96) (width 0.2) (layer "B.Cu") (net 8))
 (segment (start 115.824 60.96) (end 104.648 72.136) (width 0.2) (layer "B.Cu") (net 8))
 (segment (start 91.358 68.834) (end 91.358 70.022) (width 0.2) (layer "F.Cu") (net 4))
 (segment (start 91.358 70.022) (end 92.456 71.12) (width 0.2) (layer "F.Cu") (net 4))
 (segment (start 71.628 69.267) (end 71.68 69.215) (width 0.2) (layer "F.Cu") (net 4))
 (segment (start 92.035 79.161) (end 92.035 81.707) (width 0.2) (layer "F.Cu") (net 4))
 (segment (start 92.456 71.12) (end 92.456 78.74) (width 0.2) (layer "F.Cu") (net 4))
 (segment (start 92.456 78.74) (end 92.035 79.161) (width 0.2) (layer "F.Cu") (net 4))
 (segment (start 71.628 71.882) (end 71.628 69.267) (width 0.2) (layer "F.Cu") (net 4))
 (via (at 71.628 71.882) (size 0.6) (drill 0.3) (layers "F.Cu" "B.Cu") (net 4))
 (segment (start 92.035 81.707) (end 90.43 83.312) (width 0.2) (layer "B.Cu") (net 4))
 (segment (start 72.644 82.804) (end 72.644 72.898) (width 0.2) (layer "B.Cu") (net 4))
 (segment (start 73.152 83.312) (end 72.644 82.804) (width 0.2) (layer "B.Cu") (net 4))
 (segment (start 90.43 83.312) (end 73.152 83.312) (width 0.2) (layer "B.Cu") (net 4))
 (segment (start 71.628 71.882) (end 72.644 72.898) (width 0.2) (layer "B.Cu") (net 4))
 (segment (start 83.82 63.5) (end 83.312 63.5) (width 0.635) (layer "F.Cu") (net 3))
 (segment (start 99.62 69.925) (end 96.69 72.855) (width 0.635) (layer "F.Cu") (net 3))
 (segment (start 121.158 69.9008) (end 114.3242 69.9008) (width 0.2) (layer "F.Cu") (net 3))
 (segment (start 114.3 69.925) (end 99.62 69.925) (width 0.635) (layer "F.Cu") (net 3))
 (segment (start 96.69 74.93) (end 96.69 78.355) (width 0.635) (layer "F.Cu") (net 3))
 (segment (start 121.158 69.9008) (end 122.5804 69.9008) (width 0.2) (layer "F.Cu") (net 3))
 (segment (start 122.5804 69.9008) (end 125.095 72.4154) (width 0.2) (layer "F.Cu") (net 3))
 (segment (start 84.415 62.905) (end 83.82 63.5) (width 0.635) (layer "F.Cu") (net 3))
 (segment (start 84.415 62.484) (end 84.328 62.484) (width 0.635) (layer "F.Cu") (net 3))
 (segment (start 84.415 58.847) (end 84.415 62.484) (width 0.635) (layer "F.Cu") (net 3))
 (segment (start 96.69 72.855) (end 96.69 74.93) (width 0.635) (layer "F.Cu") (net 3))
 (segment (start 84.415 64.603) (end 84.415 65.024) (width 0.635) (layer "F.Cu") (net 3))
 (segment (start 96.69 78.355) (end 97.115 78.78) (width 0.635) (layer "F.Cu") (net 3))
 (segment (start 83.312 63.5) (end 84.415 64.603) (width 0.635) (layer "F.Cu") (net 3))
 (segment (start 84.328 64.008) (end 83.82 63.5) (width 0.635) (layer "F.Cu") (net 3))
 (segment (start 84.415 62.484) (end 84.415 62.905) (width 0.635) (layer "F.Cu") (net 3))
 (segment (start 84.328 62.484) (end 83.312 63.5) (width 0.635) (layer "F.Cu") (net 3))
 (segment (start 97.115 81.707) (end 97.115 78.78) (width 0.635) (layer "F.Cu") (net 3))
 (segment (start 84.415 62.905) (end 84.415 65.024) (width 0.635) (layer "F.Cu") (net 3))
 (segment (start 83.312 63.5) (end 82.296 63.5) (width 0.635) (layer "F.Cu") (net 3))
 (segment (start 84.415 64.008) (end 84.328 64.008) (width 0.635) (layer "F.Cu") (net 3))
 (segment (start 114.3242 69.9008) (end 114.3 69.925) (width 0.2) (layer "F.Cu") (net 3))
 (via (at 84.415 62.905) (size 0.6) (drill 0.3) (layers "F.Cu" "B.Cu") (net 3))
 (via (at 84.415 64.008) (size 0.6) (drill 0.3) (layers "F.Cu" "B.Cu") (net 3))
 (via (at 84.415 65.024) (size 0.6) (drill 0.3) (layers "F.Cu" "B.Cu") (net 3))
 (segment (start 97.115 81.707) (end 97.115 78.7) (width 0.635) (layer "B.Cu") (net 3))
 (segment (start 84.415 76.2) (end 84.415 64.008) (width 0.635) (layer "B.Cu") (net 3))
 (segment (start 75.2475 77.7875) (end 82.8275 77.7875) (width 0.635) (layer "B.Cu") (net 3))
 (segment (start 86.0025 77.7875) (end 84.415 76.2) (width 0.635) (layer "B.Cu") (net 3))
 (segment (start 74.255 78.78) (end 75.2475 77.7875) (width 0.635) (layer "B.Cu") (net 3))
 (segment (start 97.115 78.7) (end 96.2025 77.7875) (width 0.635) (layer "B.Cu") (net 3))
 (segment (start 74.255 81.707) (end 74.255 78.78) (width 0.635) (layer "B.Cu") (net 3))
 (segment (start 86.0025 77.7875) (end 96.2025 77.7875) (width 0.635) (layer "B.Cu") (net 3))
 (segment (start 82.8275 77.7875) (end 84.415 76.2) (width 0.635) (layer "B.Cu") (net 3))
 (segment (start 84.415 63.5) (end 84.415 62.905) (width 0.635) (layer "B.Cu") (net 3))
 (segment (start 84.415 64.008) (end 84.415 63.5) (width 0.635) (layer "B.Cu") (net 3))
 (segment (start 119.484 82.804) (end 125.984 82.804) (width 0.2) (layer "F.Cu") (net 12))
 (segment (start 116.586 77.542) (end 114.3 75.256) (width 0.2) (layer "F.Cu") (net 12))
 (segment (start 114.3 75.256) (end 114.3 73.025) (width 0.2) (layer "F.Cu") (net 12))
 (segment (start 111.252 83.312) (end 116.078 83.312) (width 0.2) (layer "F.Cu") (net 12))
 (segment (start 116.586 82.804) (end 116.586 77.542) (width 0.2) (layer "F.Cu") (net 12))
 (segment (start 89.495 81.707) (end 91.1 83.312) (width 0.2) (layer "F.Cu") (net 12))
 (segment (start 116.586 82.804) (end 116.078 83.312) (width 0.2) (layer "F.Cu") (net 12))
 (segment (start 91.1 83.312) (end 111.252 83.312) (width 0.2) (layer "F.Cu") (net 12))
 (segment (start 119.484 82.804) (end 116.586 82.804) (width 0.2) (layer "F.Cu") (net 12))
 (segment (start 91.948 72.39) (end 91.948 77.47) (width 0.2) (layer "F.Cu") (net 7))
 (segment (start 90.678 78.74) (end 83.312 78.74) (width 0.2) (layer "F.Cu") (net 7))
 (segment (start 91.948 77.47) (end 90.678 78.74) (width 0.2) (layer "F.Cu") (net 7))
 (segment (start 90.708 71.15) (end 91.948 72.39) (width 0.2) (layer "F.Cu") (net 7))
 (segment (start 83.312 78.74) (end 81.875 80.177) (width 0.2) (layer "F.Cu") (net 7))
 (segment (start 81.875 80.177) (end 81.875 81.707) (width 0.2) (layer "F.Cu") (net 7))
 (segment (start 90.708 68.834) (end 90.708 71.15) (width 0.2) (layer "F.Cu") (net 7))
 (segment (start 125.095 67.3354) (end 126.492 68.7324) (width 0.2) (layer "F.Cu") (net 6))
 (segment (start 125.984 73.66) (end 122.4788 73.66) (width 0.2) (layer "F.Cu") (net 6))
 (segment (start 122.4788 73.66) (end 121.158 74.9808) (width 0.2) (layer "F.Cu") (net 6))
 (segment (start 126.492 68.7324) (end 126.492 73.152) (width 0.2) (layer "F.Cu") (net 6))
 (segment (start 126.492 73.152) (end 125.984 73.66) (width 0.2) (layer "F.Cu") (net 6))
 (segment (start 104.735 81.707) (end 104.735 79.161) (width 0.2) (layer "B.Cu") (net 6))
 (segment (start 104.735 79.161) (end 115.316 68.58) (width 0.2) (layer "B.Cu") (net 6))
 (segment (start 123.8504 68.58) (end 125.095 67.3354) (width 0.2) (layer "B.Cu") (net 6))
 (segment (start 115.316 68.58) (end 123.8504 68.58) (width 0.2) (layer "B.Cu") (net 6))
 (segment (start 123.7234 69.8754) (end 121.158 72.4408) (width 0.2) (layer "B.Cu") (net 5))
 (segment (start 125.095 69.8754) (end 123.7234 69.8754) (width 0.2) (layer "B.Cu") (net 5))
 (segment (start 114.2492 72.4408) (end 113.665 73.025) (width 0.2) (layer "B.Cu") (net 5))
 (segment (start 121.158 72.4408) (end 114.2492 72.4408) (width 0.2) (layer "B.Cu") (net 5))
 (segment (start 107.275 79.415) (end 113.665 73.025) (width 0.2) (layer "B.Cu") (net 5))
 (segment (start 107.275 81.707) (end 107.275 79.415) (width 0.2) (layer "B.Cu") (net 5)))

